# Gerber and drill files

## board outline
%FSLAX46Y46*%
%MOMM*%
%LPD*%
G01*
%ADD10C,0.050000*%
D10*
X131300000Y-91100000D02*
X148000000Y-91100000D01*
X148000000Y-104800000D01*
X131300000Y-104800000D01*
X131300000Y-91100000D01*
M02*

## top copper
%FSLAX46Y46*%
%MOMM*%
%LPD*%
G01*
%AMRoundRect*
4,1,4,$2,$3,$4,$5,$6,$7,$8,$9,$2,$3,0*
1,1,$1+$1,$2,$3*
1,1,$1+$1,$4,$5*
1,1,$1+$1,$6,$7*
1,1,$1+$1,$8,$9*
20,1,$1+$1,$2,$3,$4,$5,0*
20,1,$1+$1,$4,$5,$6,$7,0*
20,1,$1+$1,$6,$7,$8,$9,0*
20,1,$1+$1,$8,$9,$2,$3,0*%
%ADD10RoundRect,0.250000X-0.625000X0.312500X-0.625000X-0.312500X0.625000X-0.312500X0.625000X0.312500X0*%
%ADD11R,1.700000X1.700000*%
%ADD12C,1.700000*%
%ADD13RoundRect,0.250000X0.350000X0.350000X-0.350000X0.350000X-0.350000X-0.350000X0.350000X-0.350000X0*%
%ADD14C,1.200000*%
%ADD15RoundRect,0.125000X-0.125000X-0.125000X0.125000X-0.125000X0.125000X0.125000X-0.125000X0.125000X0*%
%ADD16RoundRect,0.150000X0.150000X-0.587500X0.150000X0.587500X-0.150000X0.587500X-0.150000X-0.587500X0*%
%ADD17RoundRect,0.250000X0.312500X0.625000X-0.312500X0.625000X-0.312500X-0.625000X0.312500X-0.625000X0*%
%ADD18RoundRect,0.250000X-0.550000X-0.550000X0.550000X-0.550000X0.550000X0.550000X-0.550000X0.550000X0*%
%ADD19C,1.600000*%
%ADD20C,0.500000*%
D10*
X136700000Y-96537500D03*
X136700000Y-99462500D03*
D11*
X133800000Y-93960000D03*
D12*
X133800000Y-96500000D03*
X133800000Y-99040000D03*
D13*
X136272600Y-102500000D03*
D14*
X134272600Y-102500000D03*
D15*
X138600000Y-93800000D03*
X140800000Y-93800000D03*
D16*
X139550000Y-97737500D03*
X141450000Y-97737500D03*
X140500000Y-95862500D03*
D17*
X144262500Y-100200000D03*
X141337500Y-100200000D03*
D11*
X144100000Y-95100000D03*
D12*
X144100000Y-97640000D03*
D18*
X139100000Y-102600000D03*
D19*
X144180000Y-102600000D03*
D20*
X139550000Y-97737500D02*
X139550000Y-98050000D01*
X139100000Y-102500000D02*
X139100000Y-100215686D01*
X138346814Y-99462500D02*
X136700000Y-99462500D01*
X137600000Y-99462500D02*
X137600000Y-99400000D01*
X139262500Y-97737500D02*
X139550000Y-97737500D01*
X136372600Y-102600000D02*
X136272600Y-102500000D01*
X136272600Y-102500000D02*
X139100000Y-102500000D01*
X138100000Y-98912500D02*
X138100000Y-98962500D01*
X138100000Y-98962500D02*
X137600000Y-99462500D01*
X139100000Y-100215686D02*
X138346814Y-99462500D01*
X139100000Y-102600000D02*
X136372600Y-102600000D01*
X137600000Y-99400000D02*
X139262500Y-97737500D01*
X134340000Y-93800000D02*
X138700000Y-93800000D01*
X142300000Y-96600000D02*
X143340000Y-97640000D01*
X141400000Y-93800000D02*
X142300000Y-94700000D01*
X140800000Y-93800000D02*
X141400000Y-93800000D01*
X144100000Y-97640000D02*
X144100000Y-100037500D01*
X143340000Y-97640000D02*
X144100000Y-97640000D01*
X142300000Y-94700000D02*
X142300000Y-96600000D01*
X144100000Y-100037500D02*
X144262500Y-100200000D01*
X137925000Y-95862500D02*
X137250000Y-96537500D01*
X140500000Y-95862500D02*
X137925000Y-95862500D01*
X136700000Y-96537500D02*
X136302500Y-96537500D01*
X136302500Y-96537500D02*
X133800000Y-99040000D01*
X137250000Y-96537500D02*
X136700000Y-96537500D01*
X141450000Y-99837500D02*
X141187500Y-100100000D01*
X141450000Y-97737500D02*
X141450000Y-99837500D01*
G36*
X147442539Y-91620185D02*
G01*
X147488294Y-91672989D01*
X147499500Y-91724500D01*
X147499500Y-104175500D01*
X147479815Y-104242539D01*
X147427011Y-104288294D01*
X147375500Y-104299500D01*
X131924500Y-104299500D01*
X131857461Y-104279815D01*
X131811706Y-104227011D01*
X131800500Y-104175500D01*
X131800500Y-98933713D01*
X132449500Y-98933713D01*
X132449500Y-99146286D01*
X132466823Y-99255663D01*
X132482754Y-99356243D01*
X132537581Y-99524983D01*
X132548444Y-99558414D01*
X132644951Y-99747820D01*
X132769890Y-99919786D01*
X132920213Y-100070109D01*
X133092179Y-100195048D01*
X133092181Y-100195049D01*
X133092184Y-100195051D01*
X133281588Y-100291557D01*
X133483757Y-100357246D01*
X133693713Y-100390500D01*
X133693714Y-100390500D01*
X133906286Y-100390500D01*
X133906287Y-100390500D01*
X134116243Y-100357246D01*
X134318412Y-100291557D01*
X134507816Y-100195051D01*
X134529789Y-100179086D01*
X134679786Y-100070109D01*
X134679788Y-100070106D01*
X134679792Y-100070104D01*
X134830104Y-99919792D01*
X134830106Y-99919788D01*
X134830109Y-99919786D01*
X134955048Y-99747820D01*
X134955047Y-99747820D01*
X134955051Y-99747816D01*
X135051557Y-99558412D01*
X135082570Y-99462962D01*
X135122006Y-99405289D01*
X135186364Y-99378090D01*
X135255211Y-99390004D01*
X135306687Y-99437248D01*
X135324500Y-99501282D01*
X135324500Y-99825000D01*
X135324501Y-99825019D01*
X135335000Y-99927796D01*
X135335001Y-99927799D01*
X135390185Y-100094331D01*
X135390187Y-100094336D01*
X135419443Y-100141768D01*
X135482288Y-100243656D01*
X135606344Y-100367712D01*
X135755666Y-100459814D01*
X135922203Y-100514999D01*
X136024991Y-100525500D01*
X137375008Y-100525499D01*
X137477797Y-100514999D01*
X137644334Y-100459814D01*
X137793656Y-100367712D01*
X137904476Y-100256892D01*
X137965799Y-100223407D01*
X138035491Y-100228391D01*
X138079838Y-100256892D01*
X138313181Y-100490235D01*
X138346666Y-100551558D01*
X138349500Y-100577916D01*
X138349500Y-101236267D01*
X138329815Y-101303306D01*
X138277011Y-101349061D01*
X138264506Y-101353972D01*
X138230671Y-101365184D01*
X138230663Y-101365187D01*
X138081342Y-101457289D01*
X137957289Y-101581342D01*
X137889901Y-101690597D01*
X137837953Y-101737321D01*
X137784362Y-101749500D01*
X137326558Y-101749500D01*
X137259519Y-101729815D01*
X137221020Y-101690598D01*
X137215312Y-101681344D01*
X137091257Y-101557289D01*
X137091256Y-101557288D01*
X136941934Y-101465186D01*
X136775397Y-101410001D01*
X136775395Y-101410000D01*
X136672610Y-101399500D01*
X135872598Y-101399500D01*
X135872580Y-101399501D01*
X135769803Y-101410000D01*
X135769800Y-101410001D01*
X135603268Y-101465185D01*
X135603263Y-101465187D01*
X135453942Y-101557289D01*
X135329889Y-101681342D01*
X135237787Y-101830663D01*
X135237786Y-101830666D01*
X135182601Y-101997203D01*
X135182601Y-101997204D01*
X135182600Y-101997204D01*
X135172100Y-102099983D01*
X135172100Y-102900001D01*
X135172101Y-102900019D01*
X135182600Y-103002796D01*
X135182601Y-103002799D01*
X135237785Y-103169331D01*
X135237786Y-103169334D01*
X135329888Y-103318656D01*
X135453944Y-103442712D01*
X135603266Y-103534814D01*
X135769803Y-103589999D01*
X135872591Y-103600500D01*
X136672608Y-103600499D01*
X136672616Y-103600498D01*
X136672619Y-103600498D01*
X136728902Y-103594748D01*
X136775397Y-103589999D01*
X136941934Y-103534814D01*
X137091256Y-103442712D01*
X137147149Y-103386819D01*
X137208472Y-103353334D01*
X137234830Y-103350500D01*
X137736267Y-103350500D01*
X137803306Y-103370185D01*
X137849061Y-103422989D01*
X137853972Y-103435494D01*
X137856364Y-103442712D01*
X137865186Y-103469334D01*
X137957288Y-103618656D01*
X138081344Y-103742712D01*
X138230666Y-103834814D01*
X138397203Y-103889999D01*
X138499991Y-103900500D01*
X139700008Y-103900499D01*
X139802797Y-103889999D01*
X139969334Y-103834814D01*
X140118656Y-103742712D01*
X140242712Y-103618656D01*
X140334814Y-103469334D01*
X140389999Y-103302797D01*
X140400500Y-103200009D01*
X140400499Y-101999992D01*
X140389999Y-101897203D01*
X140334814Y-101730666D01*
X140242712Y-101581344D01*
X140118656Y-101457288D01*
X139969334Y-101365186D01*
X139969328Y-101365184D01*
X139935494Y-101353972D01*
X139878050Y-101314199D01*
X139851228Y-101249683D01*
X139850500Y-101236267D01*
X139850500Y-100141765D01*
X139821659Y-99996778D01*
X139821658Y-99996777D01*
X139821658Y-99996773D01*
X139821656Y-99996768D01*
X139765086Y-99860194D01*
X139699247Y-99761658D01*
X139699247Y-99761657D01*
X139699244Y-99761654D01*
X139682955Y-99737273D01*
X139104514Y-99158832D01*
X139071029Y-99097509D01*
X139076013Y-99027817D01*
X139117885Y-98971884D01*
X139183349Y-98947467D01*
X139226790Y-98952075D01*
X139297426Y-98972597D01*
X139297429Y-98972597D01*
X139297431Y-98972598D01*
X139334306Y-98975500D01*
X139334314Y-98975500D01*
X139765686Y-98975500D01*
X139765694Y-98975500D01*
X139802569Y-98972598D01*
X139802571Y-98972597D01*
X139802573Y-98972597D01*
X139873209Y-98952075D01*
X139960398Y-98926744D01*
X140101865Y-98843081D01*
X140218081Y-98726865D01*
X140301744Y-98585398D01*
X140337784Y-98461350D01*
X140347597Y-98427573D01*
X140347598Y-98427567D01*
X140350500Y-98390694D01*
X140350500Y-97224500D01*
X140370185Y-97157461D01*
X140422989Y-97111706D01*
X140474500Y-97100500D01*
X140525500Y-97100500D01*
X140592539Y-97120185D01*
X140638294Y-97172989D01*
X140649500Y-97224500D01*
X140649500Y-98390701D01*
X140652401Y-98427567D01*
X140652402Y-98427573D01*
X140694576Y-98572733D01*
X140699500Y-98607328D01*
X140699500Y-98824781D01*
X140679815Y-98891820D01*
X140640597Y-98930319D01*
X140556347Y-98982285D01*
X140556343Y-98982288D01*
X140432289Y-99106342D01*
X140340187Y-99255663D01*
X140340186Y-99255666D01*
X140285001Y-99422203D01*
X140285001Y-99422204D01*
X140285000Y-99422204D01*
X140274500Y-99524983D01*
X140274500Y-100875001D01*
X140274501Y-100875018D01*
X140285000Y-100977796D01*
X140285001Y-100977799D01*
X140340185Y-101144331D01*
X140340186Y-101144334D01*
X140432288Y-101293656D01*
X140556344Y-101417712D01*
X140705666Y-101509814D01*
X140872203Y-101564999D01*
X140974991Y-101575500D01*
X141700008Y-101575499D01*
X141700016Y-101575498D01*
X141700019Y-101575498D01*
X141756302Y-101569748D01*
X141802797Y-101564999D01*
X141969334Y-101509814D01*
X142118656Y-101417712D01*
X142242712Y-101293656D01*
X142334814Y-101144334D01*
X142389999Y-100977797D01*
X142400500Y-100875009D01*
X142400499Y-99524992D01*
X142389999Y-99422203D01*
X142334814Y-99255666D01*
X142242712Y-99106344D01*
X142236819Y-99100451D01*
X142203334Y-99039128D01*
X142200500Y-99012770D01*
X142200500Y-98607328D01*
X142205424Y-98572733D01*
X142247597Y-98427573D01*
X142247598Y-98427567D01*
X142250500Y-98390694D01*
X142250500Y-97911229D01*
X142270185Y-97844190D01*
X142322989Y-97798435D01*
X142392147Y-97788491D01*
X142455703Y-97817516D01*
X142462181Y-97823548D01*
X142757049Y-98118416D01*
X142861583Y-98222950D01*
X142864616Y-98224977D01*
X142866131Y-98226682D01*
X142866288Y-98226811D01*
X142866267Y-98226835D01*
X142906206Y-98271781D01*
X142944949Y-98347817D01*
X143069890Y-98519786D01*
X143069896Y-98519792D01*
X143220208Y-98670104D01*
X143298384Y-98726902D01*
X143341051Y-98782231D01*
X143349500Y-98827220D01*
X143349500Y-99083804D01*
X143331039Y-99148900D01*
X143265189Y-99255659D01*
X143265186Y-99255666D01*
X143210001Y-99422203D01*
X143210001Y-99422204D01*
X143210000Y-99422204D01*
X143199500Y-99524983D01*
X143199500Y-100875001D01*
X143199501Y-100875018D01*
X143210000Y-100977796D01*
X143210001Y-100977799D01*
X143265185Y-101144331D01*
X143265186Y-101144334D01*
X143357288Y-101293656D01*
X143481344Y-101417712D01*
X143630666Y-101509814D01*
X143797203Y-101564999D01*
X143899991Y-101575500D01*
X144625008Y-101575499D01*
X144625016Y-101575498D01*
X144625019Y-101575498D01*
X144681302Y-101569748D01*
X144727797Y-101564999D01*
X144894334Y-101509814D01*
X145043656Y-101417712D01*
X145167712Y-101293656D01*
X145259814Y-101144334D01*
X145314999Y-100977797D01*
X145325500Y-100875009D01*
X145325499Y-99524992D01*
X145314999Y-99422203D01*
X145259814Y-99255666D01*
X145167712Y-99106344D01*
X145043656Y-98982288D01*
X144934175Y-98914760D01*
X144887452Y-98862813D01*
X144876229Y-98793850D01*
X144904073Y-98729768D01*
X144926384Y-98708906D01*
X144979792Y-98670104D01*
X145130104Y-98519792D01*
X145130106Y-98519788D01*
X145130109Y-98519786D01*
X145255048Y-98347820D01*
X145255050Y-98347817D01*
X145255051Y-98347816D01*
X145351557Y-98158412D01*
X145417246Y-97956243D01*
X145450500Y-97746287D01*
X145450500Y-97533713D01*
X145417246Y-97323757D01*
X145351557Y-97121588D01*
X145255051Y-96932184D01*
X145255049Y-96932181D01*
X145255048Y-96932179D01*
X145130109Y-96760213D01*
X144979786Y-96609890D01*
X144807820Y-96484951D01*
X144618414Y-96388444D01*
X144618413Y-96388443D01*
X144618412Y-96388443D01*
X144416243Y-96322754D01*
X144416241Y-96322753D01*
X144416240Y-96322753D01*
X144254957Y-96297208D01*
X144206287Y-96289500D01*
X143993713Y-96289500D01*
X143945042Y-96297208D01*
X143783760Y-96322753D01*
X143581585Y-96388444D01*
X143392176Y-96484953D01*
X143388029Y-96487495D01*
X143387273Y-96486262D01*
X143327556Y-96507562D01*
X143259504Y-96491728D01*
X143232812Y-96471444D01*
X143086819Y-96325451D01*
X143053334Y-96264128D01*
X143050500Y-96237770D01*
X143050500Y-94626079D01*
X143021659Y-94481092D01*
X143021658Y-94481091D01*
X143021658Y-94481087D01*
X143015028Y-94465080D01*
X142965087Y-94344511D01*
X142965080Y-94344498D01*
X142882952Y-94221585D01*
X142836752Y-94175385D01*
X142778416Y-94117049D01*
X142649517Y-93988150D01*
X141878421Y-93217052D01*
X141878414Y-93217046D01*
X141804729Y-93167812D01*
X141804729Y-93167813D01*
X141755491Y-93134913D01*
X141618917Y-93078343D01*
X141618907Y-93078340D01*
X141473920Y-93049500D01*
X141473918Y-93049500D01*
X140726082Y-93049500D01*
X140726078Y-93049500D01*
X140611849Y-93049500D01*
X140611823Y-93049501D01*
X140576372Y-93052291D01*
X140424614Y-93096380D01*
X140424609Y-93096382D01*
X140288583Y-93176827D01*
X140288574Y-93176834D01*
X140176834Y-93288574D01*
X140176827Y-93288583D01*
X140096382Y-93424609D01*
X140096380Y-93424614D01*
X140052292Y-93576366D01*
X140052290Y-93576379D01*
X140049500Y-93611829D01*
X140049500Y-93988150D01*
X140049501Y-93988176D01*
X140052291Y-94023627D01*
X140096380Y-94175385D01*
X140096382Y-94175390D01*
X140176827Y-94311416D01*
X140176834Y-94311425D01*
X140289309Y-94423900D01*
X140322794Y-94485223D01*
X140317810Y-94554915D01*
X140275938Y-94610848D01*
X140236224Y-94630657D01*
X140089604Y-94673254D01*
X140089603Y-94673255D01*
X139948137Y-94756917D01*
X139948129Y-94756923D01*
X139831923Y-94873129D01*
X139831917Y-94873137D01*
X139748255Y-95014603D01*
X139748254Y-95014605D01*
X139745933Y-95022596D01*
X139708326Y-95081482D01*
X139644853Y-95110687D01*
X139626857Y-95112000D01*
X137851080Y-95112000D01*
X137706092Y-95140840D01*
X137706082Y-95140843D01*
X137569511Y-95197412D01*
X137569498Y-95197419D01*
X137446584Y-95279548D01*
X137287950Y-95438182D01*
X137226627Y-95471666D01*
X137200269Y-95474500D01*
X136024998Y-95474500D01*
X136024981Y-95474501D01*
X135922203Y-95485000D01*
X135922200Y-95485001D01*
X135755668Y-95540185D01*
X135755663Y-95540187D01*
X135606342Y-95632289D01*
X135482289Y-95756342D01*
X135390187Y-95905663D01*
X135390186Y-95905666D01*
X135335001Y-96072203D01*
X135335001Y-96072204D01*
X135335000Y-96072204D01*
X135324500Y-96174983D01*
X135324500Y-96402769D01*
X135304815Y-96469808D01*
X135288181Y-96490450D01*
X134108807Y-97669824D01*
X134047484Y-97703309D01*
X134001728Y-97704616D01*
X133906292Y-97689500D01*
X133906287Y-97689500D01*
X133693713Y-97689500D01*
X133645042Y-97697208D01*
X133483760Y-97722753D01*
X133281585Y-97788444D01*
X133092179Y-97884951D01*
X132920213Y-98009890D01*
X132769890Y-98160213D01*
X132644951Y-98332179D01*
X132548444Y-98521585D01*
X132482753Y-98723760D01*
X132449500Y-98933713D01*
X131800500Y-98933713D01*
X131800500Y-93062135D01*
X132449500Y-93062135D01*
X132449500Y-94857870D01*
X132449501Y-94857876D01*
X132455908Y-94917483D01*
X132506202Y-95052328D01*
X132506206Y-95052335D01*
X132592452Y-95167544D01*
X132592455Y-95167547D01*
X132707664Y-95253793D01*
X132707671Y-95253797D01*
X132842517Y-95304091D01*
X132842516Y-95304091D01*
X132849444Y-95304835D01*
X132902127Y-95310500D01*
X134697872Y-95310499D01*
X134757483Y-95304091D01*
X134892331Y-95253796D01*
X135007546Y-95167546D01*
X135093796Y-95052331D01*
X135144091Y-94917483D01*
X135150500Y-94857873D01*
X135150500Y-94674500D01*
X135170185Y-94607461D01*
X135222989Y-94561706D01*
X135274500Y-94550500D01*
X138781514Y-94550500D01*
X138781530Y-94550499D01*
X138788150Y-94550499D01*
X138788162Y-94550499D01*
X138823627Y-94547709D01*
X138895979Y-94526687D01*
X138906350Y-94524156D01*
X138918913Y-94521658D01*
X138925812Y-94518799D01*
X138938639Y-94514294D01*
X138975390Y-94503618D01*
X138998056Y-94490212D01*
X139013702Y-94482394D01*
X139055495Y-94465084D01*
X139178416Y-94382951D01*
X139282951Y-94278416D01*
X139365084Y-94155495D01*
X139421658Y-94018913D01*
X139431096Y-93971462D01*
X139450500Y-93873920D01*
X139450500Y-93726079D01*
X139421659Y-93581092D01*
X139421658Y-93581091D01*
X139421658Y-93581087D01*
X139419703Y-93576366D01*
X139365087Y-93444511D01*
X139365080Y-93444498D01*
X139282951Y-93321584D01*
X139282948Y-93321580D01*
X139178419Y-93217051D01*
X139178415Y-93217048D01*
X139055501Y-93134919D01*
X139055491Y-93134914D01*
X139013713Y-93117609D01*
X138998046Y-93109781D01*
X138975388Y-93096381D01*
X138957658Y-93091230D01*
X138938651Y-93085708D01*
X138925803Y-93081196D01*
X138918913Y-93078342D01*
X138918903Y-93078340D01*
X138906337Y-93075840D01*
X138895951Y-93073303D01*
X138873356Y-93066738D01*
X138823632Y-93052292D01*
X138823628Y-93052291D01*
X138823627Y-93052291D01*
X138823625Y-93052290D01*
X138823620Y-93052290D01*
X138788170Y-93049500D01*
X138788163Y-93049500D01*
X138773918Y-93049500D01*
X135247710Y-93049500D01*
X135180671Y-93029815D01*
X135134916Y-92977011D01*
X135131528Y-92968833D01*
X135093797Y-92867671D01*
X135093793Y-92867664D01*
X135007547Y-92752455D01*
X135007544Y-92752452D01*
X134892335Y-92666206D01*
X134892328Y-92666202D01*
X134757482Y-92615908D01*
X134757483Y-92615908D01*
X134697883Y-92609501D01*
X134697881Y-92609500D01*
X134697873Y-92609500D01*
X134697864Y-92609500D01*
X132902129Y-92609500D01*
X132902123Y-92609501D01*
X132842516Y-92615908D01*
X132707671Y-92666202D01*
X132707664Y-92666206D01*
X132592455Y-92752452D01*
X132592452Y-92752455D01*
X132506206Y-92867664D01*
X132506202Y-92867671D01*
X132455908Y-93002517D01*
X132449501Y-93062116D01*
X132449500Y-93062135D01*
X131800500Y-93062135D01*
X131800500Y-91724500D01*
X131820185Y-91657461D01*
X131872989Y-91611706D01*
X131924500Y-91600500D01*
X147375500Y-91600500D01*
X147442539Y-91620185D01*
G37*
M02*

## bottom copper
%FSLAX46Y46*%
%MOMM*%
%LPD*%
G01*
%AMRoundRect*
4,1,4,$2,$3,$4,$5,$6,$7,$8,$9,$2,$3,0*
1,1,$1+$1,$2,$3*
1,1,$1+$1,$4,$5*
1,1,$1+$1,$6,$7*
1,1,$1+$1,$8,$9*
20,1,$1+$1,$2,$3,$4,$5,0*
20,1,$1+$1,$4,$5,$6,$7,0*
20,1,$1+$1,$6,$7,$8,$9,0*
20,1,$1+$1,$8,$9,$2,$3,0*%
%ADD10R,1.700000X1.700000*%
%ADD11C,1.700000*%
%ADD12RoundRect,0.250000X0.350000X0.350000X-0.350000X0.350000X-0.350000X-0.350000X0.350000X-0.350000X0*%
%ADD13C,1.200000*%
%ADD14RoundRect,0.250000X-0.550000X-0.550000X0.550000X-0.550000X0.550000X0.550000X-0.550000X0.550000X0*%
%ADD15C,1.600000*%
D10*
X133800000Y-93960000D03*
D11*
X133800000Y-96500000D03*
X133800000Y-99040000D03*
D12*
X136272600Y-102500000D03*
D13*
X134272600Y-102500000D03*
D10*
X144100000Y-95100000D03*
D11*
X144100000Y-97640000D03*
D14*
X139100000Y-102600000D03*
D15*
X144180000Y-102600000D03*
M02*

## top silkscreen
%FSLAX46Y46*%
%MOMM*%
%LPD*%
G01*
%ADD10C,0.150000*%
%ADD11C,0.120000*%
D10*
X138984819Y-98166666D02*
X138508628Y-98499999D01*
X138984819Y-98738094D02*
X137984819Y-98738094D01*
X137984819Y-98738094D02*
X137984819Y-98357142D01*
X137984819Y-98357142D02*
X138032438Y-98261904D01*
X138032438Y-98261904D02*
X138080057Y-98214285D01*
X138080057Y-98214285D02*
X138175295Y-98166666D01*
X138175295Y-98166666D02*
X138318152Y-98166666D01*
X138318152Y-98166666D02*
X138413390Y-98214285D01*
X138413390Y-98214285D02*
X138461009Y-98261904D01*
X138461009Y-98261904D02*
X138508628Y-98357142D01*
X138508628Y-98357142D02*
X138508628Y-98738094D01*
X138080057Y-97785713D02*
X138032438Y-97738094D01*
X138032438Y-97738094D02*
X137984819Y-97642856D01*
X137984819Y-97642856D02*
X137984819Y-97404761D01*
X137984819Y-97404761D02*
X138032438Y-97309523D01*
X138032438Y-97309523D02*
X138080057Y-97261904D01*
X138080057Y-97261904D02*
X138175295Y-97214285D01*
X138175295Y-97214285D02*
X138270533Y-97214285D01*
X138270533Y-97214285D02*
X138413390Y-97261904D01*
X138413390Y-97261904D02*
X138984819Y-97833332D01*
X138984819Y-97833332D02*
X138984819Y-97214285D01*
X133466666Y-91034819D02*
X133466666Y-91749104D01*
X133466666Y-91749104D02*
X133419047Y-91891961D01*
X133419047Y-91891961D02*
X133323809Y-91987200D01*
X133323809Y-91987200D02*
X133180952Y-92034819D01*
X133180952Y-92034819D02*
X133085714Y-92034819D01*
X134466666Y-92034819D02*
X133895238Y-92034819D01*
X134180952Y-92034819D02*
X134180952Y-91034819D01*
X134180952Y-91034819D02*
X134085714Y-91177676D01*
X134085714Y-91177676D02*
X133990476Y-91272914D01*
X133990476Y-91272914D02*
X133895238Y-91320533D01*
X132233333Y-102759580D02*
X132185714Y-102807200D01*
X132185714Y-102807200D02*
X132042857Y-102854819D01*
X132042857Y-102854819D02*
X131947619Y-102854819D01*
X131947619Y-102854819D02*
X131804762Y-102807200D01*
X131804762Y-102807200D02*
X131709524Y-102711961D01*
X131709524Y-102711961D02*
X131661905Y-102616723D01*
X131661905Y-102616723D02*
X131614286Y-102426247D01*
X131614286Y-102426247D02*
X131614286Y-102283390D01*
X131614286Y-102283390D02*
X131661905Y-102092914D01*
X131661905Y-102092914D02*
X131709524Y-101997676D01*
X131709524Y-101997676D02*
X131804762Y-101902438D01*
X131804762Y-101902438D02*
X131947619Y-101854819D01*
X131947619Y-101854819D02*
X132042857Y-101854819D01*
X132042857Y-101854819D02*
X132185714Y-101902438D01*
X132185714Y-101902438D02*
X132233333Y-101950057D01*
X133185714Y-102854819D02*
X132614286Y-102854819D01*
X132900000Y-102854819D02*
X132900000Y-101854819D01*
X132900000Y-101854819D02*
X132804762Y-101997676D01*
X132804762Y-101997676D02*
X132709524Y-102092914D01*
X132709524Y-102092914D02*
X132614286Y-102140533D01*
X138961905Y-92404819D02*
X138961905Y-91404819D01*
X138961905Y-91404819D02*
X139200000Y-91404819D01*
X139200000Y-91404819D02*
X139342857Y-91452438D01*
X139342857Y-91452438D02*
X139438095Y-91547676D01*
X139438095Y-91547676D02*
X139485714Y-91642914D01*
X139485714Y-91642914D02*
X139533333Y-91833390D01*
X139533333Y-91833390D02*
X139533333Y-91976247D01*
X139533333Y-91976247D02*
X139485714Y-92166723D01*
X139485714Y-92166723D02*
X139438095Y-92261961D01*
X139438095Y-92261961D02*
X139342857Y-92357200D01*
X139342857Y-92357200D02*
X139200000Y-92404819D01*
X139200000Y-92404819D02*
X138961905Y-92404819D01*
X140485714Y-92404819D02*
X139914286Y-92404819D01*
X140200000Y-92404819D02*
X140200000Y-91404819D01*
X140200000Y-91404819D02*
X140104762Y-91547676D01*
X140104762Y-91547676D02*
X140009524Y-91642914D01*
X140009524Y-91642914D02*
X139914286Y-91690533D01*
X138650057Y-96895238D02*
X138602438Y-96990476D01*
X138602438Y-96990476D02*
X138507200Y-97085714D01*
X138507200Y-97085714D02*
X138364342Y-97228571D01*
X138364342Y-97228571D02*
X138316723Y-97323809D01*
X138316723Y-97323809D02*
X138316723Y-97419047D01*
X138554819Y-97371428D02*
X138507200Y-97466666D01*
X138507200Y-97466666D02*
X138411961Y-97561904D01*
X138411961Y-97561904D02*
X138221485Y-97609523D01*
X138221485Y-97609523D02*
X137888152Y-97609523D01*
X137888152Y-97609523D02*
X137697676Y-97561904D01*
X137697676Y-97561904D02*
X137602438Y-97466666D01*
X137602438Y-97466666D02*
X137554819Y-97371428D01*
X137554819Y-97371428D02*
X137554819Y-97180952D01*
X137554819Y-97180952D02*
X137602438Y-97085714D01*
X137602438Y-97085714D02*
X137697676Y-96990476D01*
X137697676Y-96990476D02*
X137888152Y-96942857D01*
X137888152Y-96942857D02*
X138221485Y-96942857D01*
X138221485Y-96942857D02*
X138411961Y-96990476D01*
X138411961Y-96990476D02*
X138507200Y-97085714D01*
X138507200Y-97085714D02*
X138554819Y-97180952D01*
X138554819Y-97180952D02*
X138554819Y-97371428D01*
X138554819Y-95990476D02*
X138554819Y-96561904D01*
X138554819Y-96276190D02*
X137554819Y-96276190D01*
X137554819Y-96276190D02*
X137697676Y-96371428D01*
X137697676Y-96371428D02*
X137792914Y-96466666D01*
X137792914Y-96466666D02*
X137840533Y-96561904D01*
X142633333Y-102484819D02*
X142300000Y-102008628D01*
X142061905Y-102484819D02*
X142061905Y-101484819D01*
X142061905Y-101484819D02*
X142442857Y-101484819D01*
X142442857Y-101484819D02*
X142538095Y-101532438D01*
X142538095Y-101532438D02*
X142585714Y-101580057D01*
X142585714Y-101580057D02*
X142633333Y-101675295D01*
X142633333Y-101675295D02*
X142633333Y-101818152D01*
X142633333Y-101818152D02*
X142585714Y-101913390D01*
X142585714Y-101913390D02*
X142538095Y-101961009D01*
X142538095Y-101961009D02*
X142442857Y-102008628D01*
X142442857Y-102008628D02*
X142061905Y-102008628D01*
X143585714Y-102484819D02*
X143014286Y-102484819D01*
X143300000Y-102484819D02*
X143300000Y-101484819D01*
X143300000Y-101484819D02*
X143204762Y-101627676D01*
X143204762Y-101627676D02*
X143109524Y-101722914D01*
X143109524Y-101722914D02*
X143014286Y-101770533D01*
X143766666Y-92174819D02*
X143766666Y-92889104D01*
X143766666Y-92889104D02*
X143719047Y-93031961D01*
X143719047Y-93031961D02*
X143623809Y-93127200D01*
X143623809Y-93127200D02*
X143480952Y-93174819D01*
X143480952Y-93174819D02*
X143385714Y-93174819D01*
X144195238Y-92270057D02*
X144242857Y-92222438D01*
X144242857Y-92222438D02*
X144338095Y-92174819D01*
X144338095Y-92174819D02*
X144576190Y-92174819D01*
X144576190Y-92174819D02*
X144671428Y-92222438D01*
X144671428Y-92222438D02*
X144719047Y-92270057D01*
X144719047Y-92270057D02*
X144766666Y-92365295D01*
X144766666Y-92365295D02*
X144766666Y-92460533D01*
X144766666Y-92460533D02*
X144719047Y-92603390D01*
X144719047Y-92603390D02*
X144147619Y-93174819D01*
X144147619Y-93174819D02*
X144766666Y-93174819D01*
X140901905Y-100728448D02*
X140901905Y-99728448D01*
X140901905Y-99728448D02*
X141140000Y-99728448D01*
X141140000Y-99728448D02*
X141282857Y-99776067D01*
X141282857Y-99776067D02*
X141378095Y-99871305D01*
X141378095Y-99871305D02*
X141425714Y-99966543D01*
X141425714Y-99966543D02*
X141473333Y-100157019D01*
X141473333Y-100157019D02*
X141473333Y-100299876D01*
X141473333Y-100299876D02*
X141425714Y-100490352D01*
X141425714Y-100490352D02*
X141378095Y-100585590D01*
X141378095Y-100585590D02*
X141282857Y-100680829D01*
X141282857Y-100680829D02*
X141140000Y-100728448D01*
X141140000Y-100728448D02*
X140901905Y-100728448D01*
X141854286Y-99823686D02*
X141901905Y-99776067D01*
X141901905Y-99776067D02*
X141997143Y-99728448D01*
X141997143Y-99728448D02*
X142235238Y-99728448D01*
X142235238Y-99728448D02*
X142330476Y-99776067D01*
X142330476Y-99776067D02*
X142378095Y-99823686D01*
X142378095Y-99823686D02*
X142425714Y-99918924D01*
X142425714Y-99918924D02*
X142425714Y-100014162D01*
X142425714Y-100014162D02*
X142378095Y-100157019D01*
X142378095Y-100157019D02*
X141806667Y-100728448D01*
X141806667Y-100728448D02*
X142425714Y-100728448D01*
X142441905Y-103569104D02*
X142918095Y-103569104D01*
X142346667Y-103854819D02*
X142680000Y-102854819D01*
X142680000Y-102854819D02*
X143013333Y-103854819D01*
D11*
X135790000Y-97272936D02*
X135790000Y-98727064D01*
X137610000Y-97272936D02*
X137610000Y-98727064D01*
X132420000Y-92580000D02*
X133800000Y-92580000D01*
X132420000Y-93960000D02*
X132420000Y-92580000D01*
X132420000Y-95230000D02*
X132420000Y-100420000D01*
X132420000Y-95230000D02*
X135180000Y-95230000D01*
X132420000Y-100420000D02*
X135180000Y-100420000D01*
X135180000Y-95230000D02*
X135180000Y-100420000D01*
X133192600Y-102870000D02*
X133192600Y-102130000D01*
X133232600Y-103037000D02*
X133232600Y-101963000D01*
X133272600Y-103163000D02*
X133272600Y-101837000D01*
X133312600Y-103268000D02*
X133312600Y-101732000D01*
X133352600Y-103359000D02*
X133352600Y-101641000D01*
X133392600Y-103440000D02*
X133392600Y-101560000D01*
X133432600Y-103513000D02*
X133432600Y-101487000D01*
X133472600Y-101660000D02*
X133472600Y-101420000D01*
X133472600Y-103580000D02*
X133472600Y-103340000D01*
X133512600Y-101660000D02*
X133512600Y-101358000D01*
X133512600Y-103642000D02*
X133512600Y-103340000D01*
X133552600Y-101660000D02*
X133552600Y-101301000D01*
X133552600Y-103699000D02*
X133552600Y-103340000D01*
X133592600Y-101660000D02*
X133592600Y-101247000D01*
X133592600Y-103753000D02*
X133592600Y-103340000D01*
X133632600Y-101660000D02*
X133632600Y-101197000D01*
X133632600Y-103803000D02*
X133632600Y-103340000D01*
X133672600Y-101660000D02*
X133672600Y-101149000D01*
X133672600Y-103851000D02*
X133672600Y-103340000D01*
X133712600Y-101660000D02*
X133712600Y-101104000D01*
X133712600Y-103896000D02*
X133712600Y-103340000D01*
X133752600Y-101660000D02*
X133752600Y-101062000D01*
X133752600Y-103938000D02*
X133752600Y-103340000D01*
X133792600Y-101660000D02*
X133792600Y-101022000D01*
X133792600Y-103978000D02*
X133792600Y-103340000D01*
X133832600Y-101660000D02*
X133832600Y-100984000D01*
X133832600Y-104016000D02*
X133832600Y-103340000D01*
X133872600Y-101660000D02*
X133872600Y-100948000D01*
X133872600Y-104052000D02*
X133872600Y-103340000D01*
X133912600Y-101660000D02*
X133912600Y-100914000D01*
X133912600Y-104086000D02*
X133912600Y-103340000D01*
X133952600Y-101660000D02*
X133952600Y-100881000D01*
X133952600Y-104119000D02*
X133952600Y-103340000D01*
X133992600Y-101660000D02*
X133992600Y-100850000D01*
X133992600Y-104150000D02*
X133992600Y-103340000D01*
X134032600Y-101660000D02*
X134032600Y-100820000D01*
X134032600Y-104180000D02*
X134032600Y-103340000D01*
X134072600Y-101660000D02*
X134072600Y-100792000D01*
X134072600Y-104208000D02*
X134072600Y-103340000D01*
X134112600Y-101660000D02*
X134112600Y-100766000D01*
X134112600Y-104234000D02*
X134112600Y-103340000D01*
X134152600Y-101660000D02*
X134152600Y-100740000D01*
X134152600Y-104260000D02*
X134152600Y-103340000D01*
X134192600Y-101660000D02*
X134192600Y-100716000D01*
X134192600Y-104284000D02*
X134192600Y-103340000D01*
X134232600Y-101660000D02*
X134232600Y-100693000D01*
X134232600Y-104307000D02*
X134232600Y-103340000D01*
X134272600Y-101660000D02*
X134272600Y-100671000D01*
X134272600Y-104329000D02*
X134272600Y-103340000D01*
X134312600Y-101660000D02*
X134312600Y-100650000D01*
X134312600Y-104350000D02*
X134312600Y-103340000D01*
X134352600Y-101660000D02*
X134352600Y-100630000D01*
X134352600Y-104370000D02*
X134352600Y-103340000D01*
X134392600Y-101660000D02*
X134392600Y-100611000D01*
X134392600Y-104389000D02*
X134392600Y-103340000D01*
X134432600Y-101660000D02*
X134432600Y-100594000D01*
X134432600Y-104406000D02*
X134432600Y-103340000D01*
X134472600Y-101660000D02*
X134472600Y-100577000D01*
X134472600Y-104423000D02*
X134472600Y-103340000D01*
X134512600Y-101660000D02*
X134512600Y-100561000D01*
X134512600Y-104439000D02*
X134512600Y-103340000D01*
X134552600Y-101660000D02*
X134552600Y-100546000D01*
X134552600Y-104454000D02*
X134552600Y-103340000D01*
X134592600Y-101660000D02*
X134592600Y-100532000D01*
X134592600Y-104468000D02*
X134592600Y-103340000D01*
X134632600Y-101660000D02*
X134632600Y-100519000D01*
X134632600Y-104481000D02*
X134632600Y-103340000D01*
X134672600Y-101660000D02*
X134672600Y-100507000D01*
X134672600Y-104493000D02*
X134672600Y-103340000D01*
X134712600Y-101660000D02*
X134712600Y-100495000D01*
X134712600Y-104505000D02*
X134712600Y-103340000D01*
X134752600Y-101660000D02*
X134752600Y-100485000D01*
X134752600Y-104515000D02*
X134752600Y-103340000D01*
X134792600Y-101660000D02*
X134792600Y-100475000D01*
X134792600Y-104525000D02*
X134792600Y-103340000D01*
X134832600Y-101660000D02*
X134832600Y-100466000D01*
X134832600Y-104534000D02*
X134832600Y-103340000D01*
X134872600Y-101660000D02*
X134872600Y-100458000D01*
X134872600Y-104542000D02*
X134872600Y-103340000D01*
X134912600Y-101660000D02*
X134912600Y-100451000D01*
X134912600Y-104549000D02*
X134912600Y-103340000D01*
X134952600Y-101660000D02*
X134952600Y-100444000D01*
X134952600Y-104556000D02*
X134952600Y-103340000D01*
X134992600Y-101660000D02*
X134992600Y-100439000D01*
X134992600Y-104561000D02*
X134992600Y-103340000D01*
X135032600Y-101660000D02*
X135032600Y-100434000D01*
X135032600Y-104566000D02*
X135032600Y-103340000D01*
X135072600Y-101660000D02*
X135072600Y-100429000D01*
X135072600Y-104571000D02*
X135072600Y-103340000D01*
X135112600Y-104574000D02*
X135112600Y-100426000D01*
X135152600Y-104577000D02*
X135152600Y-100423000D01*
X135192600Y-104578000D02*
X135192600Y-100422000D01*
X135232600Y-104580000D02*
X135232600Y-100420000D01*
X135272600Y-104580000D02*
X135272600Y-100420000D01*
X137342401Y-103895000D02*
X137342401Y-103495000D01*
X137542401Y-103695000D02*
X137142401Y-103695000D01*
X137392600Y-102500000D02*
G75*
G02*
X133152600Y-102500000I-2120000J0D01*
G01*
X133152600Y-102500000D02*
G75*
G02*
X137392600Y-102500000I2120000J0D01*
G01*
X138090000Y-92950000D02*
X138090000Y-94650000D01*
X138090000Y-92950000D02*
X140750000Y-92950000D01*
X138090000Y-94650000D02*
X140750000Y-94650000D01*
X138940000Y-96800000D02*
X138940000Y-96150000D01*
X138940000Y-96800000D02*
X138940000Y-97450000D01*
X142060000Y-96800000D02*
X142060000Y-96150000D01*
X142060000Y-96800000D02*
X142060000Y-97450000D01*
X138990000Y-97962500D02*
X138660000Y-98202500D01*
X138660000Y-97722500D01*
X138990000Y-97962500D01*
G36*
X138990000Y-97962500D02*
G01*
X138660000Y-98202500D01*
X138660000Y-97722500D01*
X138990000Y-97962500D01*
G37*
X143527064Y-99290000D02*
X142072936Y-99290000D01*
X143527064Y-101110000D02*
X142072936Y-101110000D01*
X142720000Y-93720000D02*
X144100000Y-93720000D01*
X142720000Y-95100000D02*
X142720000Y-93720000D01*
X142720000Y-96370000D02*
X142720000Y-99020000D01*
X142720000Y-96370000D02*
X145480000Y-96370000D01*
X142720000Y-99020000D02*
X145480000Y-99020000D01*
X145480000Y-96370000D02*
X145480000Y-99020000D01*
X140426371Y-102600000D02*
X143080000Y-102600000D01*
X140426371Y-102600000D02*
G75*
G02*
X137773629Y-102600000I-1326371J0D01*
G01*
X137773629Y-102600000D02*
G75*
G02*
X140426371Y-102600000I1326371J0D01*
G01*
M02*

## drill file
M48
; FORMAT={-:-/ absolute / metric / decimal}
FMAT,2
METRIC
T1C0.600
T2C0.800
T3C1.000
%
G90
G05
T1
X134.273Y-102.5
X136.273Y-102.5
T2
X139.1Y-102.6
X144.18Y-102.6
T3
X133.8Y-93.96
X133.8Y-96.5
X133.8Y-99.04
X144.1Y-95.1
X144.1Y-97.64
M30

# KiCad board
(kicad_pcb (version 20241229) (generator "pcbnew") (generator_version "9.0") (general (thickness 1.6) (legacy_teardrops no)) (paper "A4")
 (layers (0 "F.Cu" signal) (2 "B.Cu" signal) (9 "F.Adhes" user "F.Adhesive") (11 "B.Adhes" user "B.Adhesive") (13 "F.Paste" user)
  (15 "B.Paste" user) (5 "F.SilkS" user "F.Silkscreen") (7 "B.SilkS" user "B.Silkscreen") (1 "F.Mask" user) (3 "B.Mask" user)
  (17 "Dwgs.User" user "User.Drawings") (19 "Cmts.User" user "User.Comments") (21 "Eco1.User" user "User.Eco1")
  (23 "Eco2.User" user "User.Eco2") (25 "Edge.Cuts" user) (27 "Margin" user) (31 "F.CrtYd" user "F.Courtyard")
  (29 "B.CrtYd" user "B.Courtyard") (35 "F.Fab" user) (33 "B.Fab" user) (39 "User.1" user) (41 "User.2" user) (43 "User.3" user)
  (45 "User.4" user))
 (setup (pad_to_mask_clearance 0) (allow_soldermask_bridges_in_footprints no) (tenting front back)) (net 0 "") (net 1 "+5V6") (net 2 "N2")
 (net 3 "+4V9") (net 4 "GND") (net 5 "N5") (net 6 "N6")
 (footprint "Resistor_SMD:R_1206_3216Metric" (layer "F.Cu") (at 136.7 98 -90)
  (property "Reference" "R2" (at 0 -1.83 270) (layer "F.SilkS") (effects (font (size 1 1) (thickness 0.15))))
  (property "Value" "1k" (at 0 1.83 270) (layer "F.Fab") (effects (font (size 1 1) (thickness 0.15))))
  (fp_line (start -0.727064 0.91) (end 0.727064 0.91) (stroke (width 0.12) (type solid)) (layer "F.SilkS"))
  (fp_line (start -0.727064 -0.91) (end 0.727064 -0.91) (stroke (width 0.12) (type solid)) (layer "F.SilkS"))
  (pad "1" smd roundrect (at -1.4625 0 270) (size 1.125 1.75) (layers "F.Cu" "F.Mask" "F.Paste") (roundrect_rratio 0.222222) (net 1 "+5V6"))
  (pad "2" smd roundrect (at 1.4625 0 270) (size 1.125 1.75) (layers "F.Cu" "F.Mask" "F.Paste") (roundrect_rratio 0.222222) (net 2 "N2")))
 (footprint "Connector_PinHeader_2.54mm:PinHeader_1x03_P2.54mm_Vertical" (layer "F.Cu") (at 133.8 93.96)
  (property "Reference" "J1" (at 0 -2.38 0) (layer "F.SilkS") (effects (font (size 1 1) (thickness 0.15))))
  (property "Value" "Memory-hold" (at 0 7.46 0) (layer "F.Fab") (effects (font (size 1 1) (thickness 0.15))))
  (fp_line (start -1.38 -1.38) (end 0 -1.38) (stroke (width 0.12) (type solid)) (layer "F.SilkS"))
  (fp_line (start -1.38 0) (end -1.38 -1.38) (stroke (width 0.12) (type solid)) (layer "F.SilkS"))
  (fp_line (start -1.38 1.27) (end -1.38 6.46) (stroke (width 0.12) (type solid)) (layer "F.SilkS"))
  (fp_line (start -1.38 1.27) (end 1.38 1.27) (stroke (width 0.12) (type solid)) (layer "F.SilkS"))
  (fp_line (start -1.38 6.46) (end 1.38 6.46) (stroke (width 0.12) (type solid)) (layer "F.SilkS"))
  (fp_line (start 1.38 1.27) (end 1.38 6.46) (stroke (width 0.12) (type solid)) (layer "F.SilkS"))
  (pad "1" thru_hole rect (at 0 0) (size 1.7 1.7) (drill 1) (layers "*.Cu" "*.Mask") (remove_unused_layers no) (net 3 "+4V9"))
  (pad "2" thru_hole circle (at 0 2.54) (size 1.7 1.7) (drill 1) (layers "*.Cu" "*.Mask") (remove_unused_layers no) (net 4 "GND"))
  (pad "3" thru_hole circle (at 0 5.08) (size 1.7 1.7) (drill 1) (layers "*.Cu" "*.Mask") (remove_unused_layers no) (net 1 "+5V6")))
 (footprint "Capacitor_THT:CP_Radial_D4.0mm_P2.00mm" (layer "F.Cu") (at 136.2726 102.5 180)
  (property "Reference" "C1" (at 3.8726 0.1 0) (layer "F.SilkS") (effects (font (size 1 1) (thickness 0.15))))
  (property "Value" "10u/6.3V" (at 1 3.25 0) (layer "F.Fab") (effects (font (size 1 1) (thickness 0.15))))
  (fp_line (start 3.08 -0.37) (end 3.08 0.37) (stroke (width 0.12) (type solid)) (layer "F.SilkS"))
  (fp_line (start 3.04 -0.537) (end 3.04 0.537) (stroke (width 0.12) (type solid)) (layer "F.SilkS"))
  (fp_line (start 3 -0.663) (end 3 0.663) (stroke (width 0.12) (type solid)) (layer "F.SilkS"))
  (fp_line (start 2.96 -0.768) (end 2.96 0.768) (stroke (width 0.12) (type solid)) (layer "F.SilkS"))
  (fp_line (start 2.92 -0.859) (end 2.92 0.859) (stroke (width 0.12) (type solid)) (layer "F.SilkS"))
  (fp_line (start 2.88 -0.94) (end 2.88 0.94) (stroke (width 0.12) (type solid)) (layer "F.SilkS"))
  (fp_line (start 2.84 -1.013) (end 2.84 1.013) (stroke (width 0.12) (type solid)) (layer "F.SilkS"))
  (fp_line (start 2.8 0.84) (end 2.8 1.08) (stroke (width 0.12) (type solid)) (layer "F.SilkS"))
  (fp_line (start 2.8 -1.08) (end 2.8 -0.84) (stroke (width 0.12) (type solid)) (layer "F.SilkS"))
  (fp_line (start 2.76 0.84) (end 2.76 1.142) (stroke (width 0.12) (type solid)) (layer "F.SilkS"))
  (fp_line (start 2.76 -1.142) (end 2.76 -0.84) (stroke (width 0.12) (type solid)) (layer "F.SilkS"))
  (fp_line (start 2.72 0.84) (end 2.72 1.199) (stroke (width 0.12) (type solid)) (layer "F.SilkS"))
  (fp_line (start 2.72 -1.199) (end 2.72 -0.84) (stroke (width 0.12) (type solid)) (layer "F.SilkS"))
  (fp_line (start 2.68 0.84) (end 2.68 1.253) (stroke (width 0.12) (type solid)) (layer "F.SilkS"))
  (fp_line (start 2.68 -1.253) (end 2.68 -0.84) (stroke (width 0.12) (type solid)) (layer "F.SilkS"))
  (fp_line (start 2.64 0.84) (end 2.64 1.303) (stroke (width 0.12) (type solid)) (layer "F.SilkS"))
  (fp_line (start 2.64 -1.303) (end 2.64 -0.84) (stroke (width 0.12) (type solid)) (layer "F.SilkS"))
  (fp_line (start 2.6 0.84) (end 2.6 1.351) (stroke (width 0.12) (type solid)) (layer "F.SilkS"))
  (fp_line (start 2.6 -1.351) (end 2.6 -0.84) (stroke (width 0.12) (type solid)) (layer "F.SilkS"))
  (fp_line (start 2.56 0.84) (end 2.56 1.396) (stroke (width 0.12) (type solid)) (layer "F.SilkS"))
  (fp_line (start 2.56 -1.396) (end 2.56 -0.84) (stroke (width 0.12) (type solid)) (layer "F.SilkS"))
  (fp_line (start 2.52 0.84) (end 2.52 1.438) (stroke (width 0.12) (type solid)) (layer "F.SilkS"))
  (fp_line (start 2.52 -1.438) (end 2.52 -0.84) (stroke (width 0.12) (type solid)) (layer "F.SilkS"))
  (fp_line (start 2.48 0.84) (end 2.48 1.478) (stroke (width 0.12) (type solid)) (layer "F.SilkS"))
  (fp_line (start 2.48 -1.478) (end 2.48 -0.84) (stroke (width 0.12) (type solid)) (layer "F.SilkS"))
  (fp_line (start 2.44 0.84) (end 2.44 1.516) (stroke (width 0.12) (type solid)) (layer "F.SilkS"))
  (fp_line (start 2.44 -1.516) (end 2.44 -0.84) (stroke (width 0.12) (type solid)) (layer "F.SilkS"))
  (fp_line (start 2.4 0.84) (end 2.4 1.552) (stroke (width 0.12) (type solid)) (layer "F.SilkS"))
  (fp_line (start 2.4 -1.552) (end 2.4 -0.84) (stroke (width 0.12) (type solid)) (layer "F.SilkS"))
  (fp_line (start 2.36 0.84) (end 2.36 1.586) (stroke (width 0.12) (type solid)) (layer "F.SilkS"))
  (fp_line (start 2.36 -1.586) (end 2.36 -0.84) (stroke (width 0.12) (type solid)) (layer "F.SilkS"))
  (fp_line (start 2.32 0.84) (end 2.32 1.619) (stroke (width 0.12) (type solid)) (layer "F.SilkS"))
  (fp_line (start 2.32 -1.619) (end 2.32 -0.84) (stroke (width 0.12) (type solid)) (layer "F.SilkS"))
  (fp_line (start 2.28 0.84) (end 2.28 1.65) (stroke (width 0.12) (type solid)) (layer "F.SilkS"))
  (fp_line (start 2.28 -1.65) (end 2.28 -0.84) (stroke (width 0.12) (type solid)) (layer "F.SilkS"))
  (fp_line (start 2.24 0.84) (end 2.24 1.68) (stroke (width 0.12) (type solid)) (layer "F.SilkS"))
  (fp_line (start 2.24 -1.68) (end 2.24 -0.84) (stroke (width 0.12) (type solid)) (layer "F.SilkS"))
  (fp_line (start 2.2 0.84) (end 2.2 1.708) (stroke (width 0.12) (type solid)) (layer "F.SilkS"))
  (fp_line (start 2.2 -1.708) (end 2.2 -0.84) (stroke (width 0.12) (type solid)) (layer "F.SilkS"))
  (fp_line (start 2.16 0.84) (end 2.16 1.734) (stroke (width 0.12) (type solid)) (layer "F.SilkS"))
  (fp_line (start 2.16 -1.734) (end 2.16 -0.84) (stroke (width 0.12) (type solid)) (layer "F.SilkS"))
  (fp_line (start 2.12 0.84) (end 2.12 1.76) (stroke (width 0.12) (type solid)) (layer "F.SilkS"))
  (fp_line (start 2.12 -1.76) (end 2.12 -0.84) (stroke (width 0.12) (type solid)) (layer "F.SilkS"))
  (fp_line (start 2.08 0.84) (end 2.08 1.784) (stroke (width 0.12) (type solid)) (layer "F.SilkS"))
  (fp_line (start 2.08 -1.784) (end 2.08 -0.84) (stroke (width 0.12) (type solid)) (layer "F.SilkS"))
  (fp_line (start 2.04 0.84) (end 2.04 1.807) (stroke (width 0.12) (type solid)) (layer "F.SilkS"))
  (fp_line (start 2.04 -1.807) (end 2.04 -0.84) (stroke (width 0.12) (type solid)) (layer "F.SilkS"))
  (fp_line (start 2 0.84) (end 2 1.829) (stroke (width 0.12) (type solid)) (layer "F.SilkS"))
  (fp_line (start 2 -1.829) (end 2 -0.84) (stroke (width 0.12) (type solid)) (layer "F.SilkS"))
  (fp_line (start 1.96 0.84) (end 1.96 1.85) (stroke (width 0.12) (type solid)) (layer "F.SilkS"))
  (fp_line (start 1.96 -1.85) (end 1.96 -0.84) (stroke (width 0.12) (type solid)) (layer "F.SilkS"))
  (fp_line (start 1.92 0.84) (end 1.92 1.87) (stroke (width 0.12) (type solid)) (layer "F.SilkS"))
  (fp_line (start 1.92 -1.87) (end 1.92 -0.84) (stroke (width 0.12) (type solid)) (layer "F.SilkS"))
  (fp_line (start 1.88 0.84) (end 1.88 1.889) (stroke (width 0.12) (type solid)) (layer "F.SilkS"))
  (fp_line (start 1.88 -1.889) (end 1.88 -0.84) (stroke (width 0.12) (type solid)) (layer "F.SilkS"))
  (fp_line (start 1.84 0.84) (end 1.84 1.906) (stroke (width 0.12) (type solid)) (layer "F.SilkS"))
  (fp_line (start 1.84 -1.906) (end 1.84 -0.84) (stroke (width 0.12) (type solid)) (layer "F.SilkS"))
  (fp_line (start 1.8 0.84) (end 1.8 1.923) (stroke (width 0.12) (type solid)) (layer "F.SilkS"))
  (fp_line (start 1.8 -1.923) (end 1.8 -0.84) (stroke (width 0.12) (type solid)) (layer "F.SilkS"))
  (fp_line (start 1.76 0.84) (end 1.76 1.939) (stroke (width 0.12) (type solid)) (layer "F.SilkS"))
  (fp_line (start 1.76 -1.939) (end 1.76 -0.84) (stroke (width 0.12) (type solid)) (layer "F.SilkS"))
  (fp_line (start 1.72 0.84) (end 1.72 1.954) (stroke (width 0.12) (type solid)) (layer "F.SilkS"))
  (fp_line (start 1.72 -1.954) (end 1.72 -0.84) (stroke (width 0.12) (type solid)) (layer "F.SilkS"))
  (fp_line (start 1.68 0.84) (end 1.68 1.968) (stroke (width 0.12) (type solid)) (layer "F.SilkS"))
  (fp_line (start 1.68 -1.968) (end 1.68 -0.84) (stroke (width 0.12) (type solid)) (layer "F.SilkS"))
  (fp_line (start 1.64 0.84) (end 1.64 1.981) (stroke (width 0.12) (type solid)) (layer "F.SilkS"))
  (fp_line (start 1.64 -1.981) (end 1.64 -0.84) (stroke (width 0.12) (type solid)) (layer "F.SilkS"))
  (fp_line (start 1.6 0.84) (end 1.6 1.993) (stroke (width 0.12) (type solid)) (layer "F.SilkS"))
  (fp_line (start 1.6 -1.993) (end 1.6 -0.84) (stroke (width 0.12) (type solid)) (layer "F.SilkS"))
  (fp_line (start 1.56 0.84) (end 1.56 2.005) (stroke (width 0.12) (type solid)) (layer "F.SilkS"))
  (fp_line (start 1.56 -2.005) (end 1.56 -0.84) (stroke (width 0.12) (type solid)) (layer "F.SilkS"))
  (fp_line (start 1.52 0.84) (end 1.52 2.015) (stroke (width 0.12) (type solid)) (layer "F.SilkS"))
  (fp_line (start 1.52 -2.015) (end 1.52 -0.84) (stroke (width 0.12) (type solid)) (layer "F.SilkS"))
  (fp_line (start 1.48 0.84) (end 1.48 2.025) (stroke (width 0.12) (type solid)) (layer "F.SilkS"))
  (fp_line (start 1.48 -2.025) (end 1.48 -0.84) (stroke (width 0.12) (type solid)) (layer "F.SilkS"))
  (fp_line (start 1.44 0.84) (end 1.44 2.034) (stroke (width 0.12) (type solid)) (layer "F.SilkS"))
  (fp_line (start 1.44 -2.034) (end 1.44 -0.84) (stroke (width 0.12) (type solid)) (layer "F.SilkS"))
  (fp_line (start 1.4 0.84) (end 1.4 2.042) (stroke (width 0.12) (type solid)) (layer "F.SilkS"))
  (fp_line (start 1.4 -2.042) (end 1.4 -0.84) (stroke (width 0.12) (type solid)) (layer "F.SilkS"))
  (fp_line (start 1.36 0.84) (end 1.36 2.049) (stroke (width 0.12) (type solid)) (layer "F.SilkS"))
  (fp_line (start 1.36 -2.049) (end 1.36 -0.84) (stroke (width 0.12) (type solid)) (layer "F.SilkS"))
  (fp_line (start 1.32 0.84) (end 1.32 2.056) (stroke (width 0.12) (type solid)) (layer "F.SilkS"))
  (fp_line (start 1.32 -2.056) (end 1.32 -0.84) (stroke (width 0.12) (type solid)) (layer "F.SilkS"))
  (fp_line (start 1.28 0.84) (end 1.28 2.061) (stroke (width 0.12) (type solid)) (layer "F.SilkS"))
  (fp_line (start 1.28 -2.061) (end 1.28 -0.84) (stroke (width 0.12) (type solid)) (layer "F.SilkS"))
  (fp_line (start 1.24 0.84) (end 1.24 2.066) (stroke (width 0.12) (type solid)) (layer "F.SilkS"))
  (fp_line (start 1.24 -2.066) (end 1.24 -0.84) (stroke (width 0.12) (type solid)) (layer "F.SilkS"))
  (fp_line (start 1.2 0.84) (end 1.2 2.071) (stroke (width 0.12) (type solid)) (layer "F.SilkS"))
  (fp_line (start 1.2 -2.071) (end 1.2 -0.84) (stroke (width 0.12) (type solid)) (layer "F.SilkS"))
  (fp_line (start 1.16 -2.074) (end 1.16 2.074) (stroke (width 0.12) (type solid)) (layer "F.SilkS"))
  (fp_line (start 1.12 -2.077) (end 1.12 2.077) (stroke (width 0.12) (type solid)) (layer "F.SilkS"))
  (fp_line (start 1.08 -2.078) (end 1.08 2.078) (stroke (width 0.12) (type solid)) (layer "F.SilkS"))
  (fp_line (start 1.04 -2.08) (end 1.04 2.08) (stroke (width 0.12) (type solid)) (layer "F.SilkS"))
  (fp_line (start 1 -2.08) (end 1 2.08) (stroke (width 0.12) (type solid)) (layer "F.SilkS"))
  (fp_line (start -1.069801 -1.395) (end -1.069801 -0.995) (stroke (width 0.12) (type solid)) (layer "F.SilkS"))
  (fp_line (start -1.269801 -1.195) (end -0.869801 -1.195) (stroke (width 0.12) (type solid)) (layer "F.SilkS"))
  (fp_circle (center 1 0) (end 3.12 0) (stroke (width 0.12) (type solid)) (fill no) (layer "F.SilkS"))
  (pad "1" thru_hole roundrect (at 0 0 180) (size 1.2 1.2) (drill 0.6) (layers "*.Cu" "*.Mask") (remove_unused_layers no)
   (roundrect_rratio 0.208333) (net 2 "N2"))
  (pad "2" thru_hole circle (at 2 0 180) (size 1.2 1.2) (drill 0.6) (layers "*.Cu" "*.Mask") (remove_unused_layers no) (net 4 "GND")))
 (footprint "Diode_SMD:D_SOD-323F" (layer "F.Cu") (at 139.7 93.8)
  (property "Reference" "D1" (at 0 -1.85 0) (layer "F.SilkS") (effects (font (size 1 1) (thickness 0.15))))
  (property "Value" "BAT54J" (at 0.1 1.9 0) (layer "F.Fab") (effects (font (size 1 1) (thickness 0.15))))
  (fp_line (start -1.61 -0.85) (end -1.61 0.85) (stroke (width 0.12) (type solid)) (layer "F.SilkS"))
  (fp_line (start -1.61 -0.85) (end 1.05 -0.85) (stroke (width 0.12) (type solid)) (layer "F.SilkS"))
  (fp_line (start -1.61 0.85) (end 1.05 0.85) (stroke (width 0.12) (type solid)) (layer "F.SilkS"))
  (pad "1" smd roundrect (at -1.1 0) (size 0.5 0.5) (layers "F.Cu" "F.Mask" "F.Paste") (roundrect_rratio 0.25) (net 3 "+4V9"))
  (pad "2" smd roundrect (at 1.1 0) (size 0.5 0.5) (layers "F.Cu" "F.Mask" "F.Paste") (roundrect_rratio 0.25) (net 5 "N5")))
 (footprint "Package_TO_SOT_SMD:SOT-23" (layer "F.Cu") (at 140.5 96.8 90)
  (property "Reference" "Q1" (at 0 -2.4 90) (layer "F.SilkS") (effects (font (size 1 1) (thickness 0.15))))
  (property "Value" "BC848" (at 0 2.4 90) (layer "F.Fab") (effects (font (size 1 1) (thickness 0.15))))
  (fp_line (start 0 -1.56) (end 0.65 -1.56) (stroke (width 0.12) (type solid)) (layer "F.SilkS"))
  (fp_line (start 0 -1.56) (end -0.65 -1.56) (stroke (width 0.12) (type solid)) (layer "F.SilkS"))
  (fp_line (start 0 1.56) (end 0.65 1.56) (stroke (width 0.12) (type solid)) (layer "F.SilkS"))
  (fp_line (start 0 1.56) (end -0.65 1.56) (stroke (width 0.12) (type solid)) (layer "F.SilkS"))
  (fp_poly (pts (xy -1.1625 -1.51) (xy -1.4025 -1.84) (xy -0.9225 -1.84)) (stroke (width 0.12) (type solid)) (fill yes) (layer "F.SilkS"))
  (pad "1" smd roundrect (at -0.9375 -0.95 90) (size 1.475 0.6) (layers "F.Cu" "F.Mask" "F.Paste") (roundrect_rratio 0.25) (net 2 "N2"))
  (pad "2" smd roundrect (at -0.9375 0.95 90) (size 1.475 0.6) (layers "F.Cu" "F.Mask" "F.Paste") (roundrect_rratio 0.25) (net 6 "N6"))
  (pad "3" smd roundrect (at 0.9375 0 90) (size 1.475 0.6) (layers "F.Cu" "F.Mask" "F.Paste") (roundrect_rratio 0.25) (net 1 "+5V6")))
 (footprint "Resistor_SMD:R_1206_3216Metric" (layer "F.Cu") (at 142.8 100.2 180)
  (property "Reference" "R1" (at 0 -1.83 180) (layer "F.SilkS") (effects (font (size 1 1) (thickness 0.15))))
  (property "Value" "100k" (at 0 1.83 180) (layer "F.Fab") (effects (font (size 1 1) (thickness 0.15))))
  (fp_line (start -0.727064 0.91) (end 0.727064 0.91) (stroke (width 0.12) (type solid)) (layer "F.SilkS"))
  (fp_line (start -0.727064 -0.91) (end 0.727064 -0.91) (stroke (width 0.12) (type solid)) (layer "F.SilkS"))
  (pad "1" smd roundrect (at -1.4625 0 180) (size 1.125 1.75) (layers "F.Cu" "F.Mask" "F.Paste") (roundrect_rratio 0.222222) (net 5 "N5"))
  (pad "2" smd roundrect (at 1.4625 0 180) (size 1.125 1.75) (layers "F.Cu" "F.Mask" "F.Paste") (roundrect_rratio 0.222222) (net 6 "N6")))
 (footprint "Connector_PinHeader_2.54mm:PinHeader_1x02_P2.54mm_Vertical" (layer "F.Cu") (at 144.1 95.1)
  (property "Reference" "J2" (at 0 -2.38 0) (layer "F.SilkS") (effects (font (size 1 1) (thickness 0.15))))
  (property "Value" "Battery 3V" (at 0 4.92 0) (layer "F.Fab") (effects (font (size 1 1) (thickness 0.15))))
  (fp_line (start -1.38 -1.38) (end 0 -1.38) (stroke (width 0.12) (type solid)) (layer "F.SilkS"))
  (fp_line (start -1.38 0) (end -1.38 -1.38) (stroke (width 0.12) (type solid)) (layer "F.SilkS"))
  (fp_line (start -1.38 1.27) (end -1.38 3.92) (stroke (width 0.12) (type solid)) (layer "F.SilkS"))
  (fp_line (start -1.38 1.27) (end 1.38 1.27) (stroke (width 0.12) (type solid)) (layer "F.SilkS"))
  (fp_line (start -1.38 3.92) (end 1.38 3.92) (stroke (width 0.12) (type solid)) (layer "F.SilkS"))
  (fp_line (start 1.38 1.27) (end 1.38 3.92) (stroke (width 0.12) (type solid)) (layer "F.SilkS"))
  (pad "1" thru_hole rect (at 0 0) (size 1.7 1.7) (drill 1) (layers "*.Cu" "*.Mask") (remove_unused_layers no) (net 4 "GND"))
  (pad "2" thru_hole circle (at 0 2.54) (size 1.7 1.7) (drill 1) (layers "*.Cu" "*.Mask") (remove_unused_layers no) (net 5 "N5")))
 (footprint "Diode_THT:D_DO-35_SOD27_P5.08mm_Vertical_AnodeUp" (layer "F.Cu") (at 139.1 102.6)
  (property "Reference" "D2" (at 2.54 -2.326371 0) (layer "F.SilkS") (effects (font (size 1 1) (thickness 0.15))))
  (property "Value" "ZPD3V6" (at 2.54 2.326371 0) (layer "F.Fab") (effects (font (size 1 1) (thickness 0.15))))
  (fp_line (start 1.326371 0) (end 3.98 0) (stroke (width 0.12) (type solid)) (layer "F.SilkS"))
  (fp_circle (center 0 0) (end 1.326371 0) (stroke (width 0.12) (type solid)) (fill no) (layer "F.SilkS"))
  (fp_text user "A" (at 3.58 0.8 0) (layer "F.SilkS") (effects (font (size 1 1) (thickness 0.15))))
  (pad "1" thru_hole roundrect (at 0 0) (size 1.6 1.6) (drill 0.8) (layers "*.Cu" "*.Mask") (remove_unused_layers no)
   (roundrect_rratio 0.15625) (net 2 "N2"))
  (pad "2" thru_hole circle (at 5.08 0) (size 1.6 1.6) (drill 0.8) (layers "*.Cu" "*.Mask") (remove_unused_layers no) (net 4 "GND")))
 (gr_rect (start 131.3 91.1) (end 148 104.8) (stroke (width 0.05) (type default)) (fill no) (layer "Edge.Cuts"))
 (segment (start 139.55 97.7375) (end 139.55 98.05) (width 0.5) (layer "F.Cu") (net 2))
 (segment (start 139.1 102.5) (end 139.1 100.215686) (width 0.5) (layer "F.Cu") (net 2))
 (segment (start 138.346814 99.4625) (end 136.7 99.4625) (width 0.5) (layer "F.Cu") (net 2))
 (segment (start 137.6 99.4625) (end 137.6 99.4) (width 0.5) (layer "F.Cu") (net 2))
 (segment (start 139.2625 97.7375) (end 139.55 97.7375) (width 0.5) (layer "F.Cu") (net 2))
 (segment (start 136.3726 102.6) (end 136.2726 102.5) (width 0.5) (layer "F.Cu") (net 2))
 (segment (start 136.2726 102.5) (end 139.1 102.5) (width 0.5) (layer "F.Cu") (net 2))
 (segment (start 138.1 98.9125) (end 138.1 98.9625) (width 0.5) (layer "F.Cu") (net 2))
 (segment (start 138.1 98.9625) (end 137.6 99.4625) (width 0.5) (layer "F.Cu") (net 2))
 (segment (start 139.1 100.215686) (end 138.346814 99.4625) (width 0.5) (layer "F.Cu") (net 2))
 (segment (start 139.1 102.6) (end 136.3726 102.6) (width 0.5) (layer "F.Cu") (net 2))
 (segment (start 137.6 99.4) (end 139.2625 97.7375) (width 0.5) (layer "F.Cu") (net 2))
 (segment (start 134.34 93.8) (end 138.7 93.8) (width 0.5) (layer "F.Cu") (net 3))
 (segment (start 142.3 96.6) (end 143.34 97.64) (width 0.5) (layer "F.Cu") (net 5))
 (segment (start 141.4 93.8) (end 142.3 94.7) (width 0.5) (layer "F.Cu") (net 5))
 (segment (start 140.8 93.8) (end 141.4 93.8) (width 0.5) (layer "F.Cu") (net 5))
 (segment (start 144.1 97.64) (end 144.1 100.0375) (width 0.5) (layer "F.Cu") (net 5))
 (segment (start 143.34 97.64) (end 144.1 97.64) (width 0.5) (layer "F.Cu") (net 5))
 (segment (start 142.3 94.7) (end 142.3 96.6) (width 0.5) (layer "F.Cu") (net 5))
 (segment (start 144.1 100.0375) (end 144.2625 100.2) (width 0.5) (layer "F.Cu") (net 5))
 (segment (start 137.925 95.8625) (end 137.25 96.5375) (width 0.5) (layer "F.Cu") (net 1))
 (segment (start 140.5 95.8625) (end 137.925 95.8625) (width 0.5) (layer "F.Cu") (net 1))
 (segment (start 136.7 96.5375) (end 136.3025 96.5375) (width 0.5) (layer "F.Cu") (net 1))
 (segment (start 136.3025 96.5375) (end 133.8 99.04) (width 0.5) (layer "F.Cu") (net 1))
 (segment (start 137.25 96.5375) (end 136.7 96.5375) (width 0.5) (layer "F.Cu") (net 1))
 (segment (start 141.45 99.8375) (end 141.1875 100.1) (width 0.5) (layer "F.Cu") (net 6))
 (segment (start 141.45 97.7375) (end 141.45 99.8375) (width 0.5) (layer "F.Cu") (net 6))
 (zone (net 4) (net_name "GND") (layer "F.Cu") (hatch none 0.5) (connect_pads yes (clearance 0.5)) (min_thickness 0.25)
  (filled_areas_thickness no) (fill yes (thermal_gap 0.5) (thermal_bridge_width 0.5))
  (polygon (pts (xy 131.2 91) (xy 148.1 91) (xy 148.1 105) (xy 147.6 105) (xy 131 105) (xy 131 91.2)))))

